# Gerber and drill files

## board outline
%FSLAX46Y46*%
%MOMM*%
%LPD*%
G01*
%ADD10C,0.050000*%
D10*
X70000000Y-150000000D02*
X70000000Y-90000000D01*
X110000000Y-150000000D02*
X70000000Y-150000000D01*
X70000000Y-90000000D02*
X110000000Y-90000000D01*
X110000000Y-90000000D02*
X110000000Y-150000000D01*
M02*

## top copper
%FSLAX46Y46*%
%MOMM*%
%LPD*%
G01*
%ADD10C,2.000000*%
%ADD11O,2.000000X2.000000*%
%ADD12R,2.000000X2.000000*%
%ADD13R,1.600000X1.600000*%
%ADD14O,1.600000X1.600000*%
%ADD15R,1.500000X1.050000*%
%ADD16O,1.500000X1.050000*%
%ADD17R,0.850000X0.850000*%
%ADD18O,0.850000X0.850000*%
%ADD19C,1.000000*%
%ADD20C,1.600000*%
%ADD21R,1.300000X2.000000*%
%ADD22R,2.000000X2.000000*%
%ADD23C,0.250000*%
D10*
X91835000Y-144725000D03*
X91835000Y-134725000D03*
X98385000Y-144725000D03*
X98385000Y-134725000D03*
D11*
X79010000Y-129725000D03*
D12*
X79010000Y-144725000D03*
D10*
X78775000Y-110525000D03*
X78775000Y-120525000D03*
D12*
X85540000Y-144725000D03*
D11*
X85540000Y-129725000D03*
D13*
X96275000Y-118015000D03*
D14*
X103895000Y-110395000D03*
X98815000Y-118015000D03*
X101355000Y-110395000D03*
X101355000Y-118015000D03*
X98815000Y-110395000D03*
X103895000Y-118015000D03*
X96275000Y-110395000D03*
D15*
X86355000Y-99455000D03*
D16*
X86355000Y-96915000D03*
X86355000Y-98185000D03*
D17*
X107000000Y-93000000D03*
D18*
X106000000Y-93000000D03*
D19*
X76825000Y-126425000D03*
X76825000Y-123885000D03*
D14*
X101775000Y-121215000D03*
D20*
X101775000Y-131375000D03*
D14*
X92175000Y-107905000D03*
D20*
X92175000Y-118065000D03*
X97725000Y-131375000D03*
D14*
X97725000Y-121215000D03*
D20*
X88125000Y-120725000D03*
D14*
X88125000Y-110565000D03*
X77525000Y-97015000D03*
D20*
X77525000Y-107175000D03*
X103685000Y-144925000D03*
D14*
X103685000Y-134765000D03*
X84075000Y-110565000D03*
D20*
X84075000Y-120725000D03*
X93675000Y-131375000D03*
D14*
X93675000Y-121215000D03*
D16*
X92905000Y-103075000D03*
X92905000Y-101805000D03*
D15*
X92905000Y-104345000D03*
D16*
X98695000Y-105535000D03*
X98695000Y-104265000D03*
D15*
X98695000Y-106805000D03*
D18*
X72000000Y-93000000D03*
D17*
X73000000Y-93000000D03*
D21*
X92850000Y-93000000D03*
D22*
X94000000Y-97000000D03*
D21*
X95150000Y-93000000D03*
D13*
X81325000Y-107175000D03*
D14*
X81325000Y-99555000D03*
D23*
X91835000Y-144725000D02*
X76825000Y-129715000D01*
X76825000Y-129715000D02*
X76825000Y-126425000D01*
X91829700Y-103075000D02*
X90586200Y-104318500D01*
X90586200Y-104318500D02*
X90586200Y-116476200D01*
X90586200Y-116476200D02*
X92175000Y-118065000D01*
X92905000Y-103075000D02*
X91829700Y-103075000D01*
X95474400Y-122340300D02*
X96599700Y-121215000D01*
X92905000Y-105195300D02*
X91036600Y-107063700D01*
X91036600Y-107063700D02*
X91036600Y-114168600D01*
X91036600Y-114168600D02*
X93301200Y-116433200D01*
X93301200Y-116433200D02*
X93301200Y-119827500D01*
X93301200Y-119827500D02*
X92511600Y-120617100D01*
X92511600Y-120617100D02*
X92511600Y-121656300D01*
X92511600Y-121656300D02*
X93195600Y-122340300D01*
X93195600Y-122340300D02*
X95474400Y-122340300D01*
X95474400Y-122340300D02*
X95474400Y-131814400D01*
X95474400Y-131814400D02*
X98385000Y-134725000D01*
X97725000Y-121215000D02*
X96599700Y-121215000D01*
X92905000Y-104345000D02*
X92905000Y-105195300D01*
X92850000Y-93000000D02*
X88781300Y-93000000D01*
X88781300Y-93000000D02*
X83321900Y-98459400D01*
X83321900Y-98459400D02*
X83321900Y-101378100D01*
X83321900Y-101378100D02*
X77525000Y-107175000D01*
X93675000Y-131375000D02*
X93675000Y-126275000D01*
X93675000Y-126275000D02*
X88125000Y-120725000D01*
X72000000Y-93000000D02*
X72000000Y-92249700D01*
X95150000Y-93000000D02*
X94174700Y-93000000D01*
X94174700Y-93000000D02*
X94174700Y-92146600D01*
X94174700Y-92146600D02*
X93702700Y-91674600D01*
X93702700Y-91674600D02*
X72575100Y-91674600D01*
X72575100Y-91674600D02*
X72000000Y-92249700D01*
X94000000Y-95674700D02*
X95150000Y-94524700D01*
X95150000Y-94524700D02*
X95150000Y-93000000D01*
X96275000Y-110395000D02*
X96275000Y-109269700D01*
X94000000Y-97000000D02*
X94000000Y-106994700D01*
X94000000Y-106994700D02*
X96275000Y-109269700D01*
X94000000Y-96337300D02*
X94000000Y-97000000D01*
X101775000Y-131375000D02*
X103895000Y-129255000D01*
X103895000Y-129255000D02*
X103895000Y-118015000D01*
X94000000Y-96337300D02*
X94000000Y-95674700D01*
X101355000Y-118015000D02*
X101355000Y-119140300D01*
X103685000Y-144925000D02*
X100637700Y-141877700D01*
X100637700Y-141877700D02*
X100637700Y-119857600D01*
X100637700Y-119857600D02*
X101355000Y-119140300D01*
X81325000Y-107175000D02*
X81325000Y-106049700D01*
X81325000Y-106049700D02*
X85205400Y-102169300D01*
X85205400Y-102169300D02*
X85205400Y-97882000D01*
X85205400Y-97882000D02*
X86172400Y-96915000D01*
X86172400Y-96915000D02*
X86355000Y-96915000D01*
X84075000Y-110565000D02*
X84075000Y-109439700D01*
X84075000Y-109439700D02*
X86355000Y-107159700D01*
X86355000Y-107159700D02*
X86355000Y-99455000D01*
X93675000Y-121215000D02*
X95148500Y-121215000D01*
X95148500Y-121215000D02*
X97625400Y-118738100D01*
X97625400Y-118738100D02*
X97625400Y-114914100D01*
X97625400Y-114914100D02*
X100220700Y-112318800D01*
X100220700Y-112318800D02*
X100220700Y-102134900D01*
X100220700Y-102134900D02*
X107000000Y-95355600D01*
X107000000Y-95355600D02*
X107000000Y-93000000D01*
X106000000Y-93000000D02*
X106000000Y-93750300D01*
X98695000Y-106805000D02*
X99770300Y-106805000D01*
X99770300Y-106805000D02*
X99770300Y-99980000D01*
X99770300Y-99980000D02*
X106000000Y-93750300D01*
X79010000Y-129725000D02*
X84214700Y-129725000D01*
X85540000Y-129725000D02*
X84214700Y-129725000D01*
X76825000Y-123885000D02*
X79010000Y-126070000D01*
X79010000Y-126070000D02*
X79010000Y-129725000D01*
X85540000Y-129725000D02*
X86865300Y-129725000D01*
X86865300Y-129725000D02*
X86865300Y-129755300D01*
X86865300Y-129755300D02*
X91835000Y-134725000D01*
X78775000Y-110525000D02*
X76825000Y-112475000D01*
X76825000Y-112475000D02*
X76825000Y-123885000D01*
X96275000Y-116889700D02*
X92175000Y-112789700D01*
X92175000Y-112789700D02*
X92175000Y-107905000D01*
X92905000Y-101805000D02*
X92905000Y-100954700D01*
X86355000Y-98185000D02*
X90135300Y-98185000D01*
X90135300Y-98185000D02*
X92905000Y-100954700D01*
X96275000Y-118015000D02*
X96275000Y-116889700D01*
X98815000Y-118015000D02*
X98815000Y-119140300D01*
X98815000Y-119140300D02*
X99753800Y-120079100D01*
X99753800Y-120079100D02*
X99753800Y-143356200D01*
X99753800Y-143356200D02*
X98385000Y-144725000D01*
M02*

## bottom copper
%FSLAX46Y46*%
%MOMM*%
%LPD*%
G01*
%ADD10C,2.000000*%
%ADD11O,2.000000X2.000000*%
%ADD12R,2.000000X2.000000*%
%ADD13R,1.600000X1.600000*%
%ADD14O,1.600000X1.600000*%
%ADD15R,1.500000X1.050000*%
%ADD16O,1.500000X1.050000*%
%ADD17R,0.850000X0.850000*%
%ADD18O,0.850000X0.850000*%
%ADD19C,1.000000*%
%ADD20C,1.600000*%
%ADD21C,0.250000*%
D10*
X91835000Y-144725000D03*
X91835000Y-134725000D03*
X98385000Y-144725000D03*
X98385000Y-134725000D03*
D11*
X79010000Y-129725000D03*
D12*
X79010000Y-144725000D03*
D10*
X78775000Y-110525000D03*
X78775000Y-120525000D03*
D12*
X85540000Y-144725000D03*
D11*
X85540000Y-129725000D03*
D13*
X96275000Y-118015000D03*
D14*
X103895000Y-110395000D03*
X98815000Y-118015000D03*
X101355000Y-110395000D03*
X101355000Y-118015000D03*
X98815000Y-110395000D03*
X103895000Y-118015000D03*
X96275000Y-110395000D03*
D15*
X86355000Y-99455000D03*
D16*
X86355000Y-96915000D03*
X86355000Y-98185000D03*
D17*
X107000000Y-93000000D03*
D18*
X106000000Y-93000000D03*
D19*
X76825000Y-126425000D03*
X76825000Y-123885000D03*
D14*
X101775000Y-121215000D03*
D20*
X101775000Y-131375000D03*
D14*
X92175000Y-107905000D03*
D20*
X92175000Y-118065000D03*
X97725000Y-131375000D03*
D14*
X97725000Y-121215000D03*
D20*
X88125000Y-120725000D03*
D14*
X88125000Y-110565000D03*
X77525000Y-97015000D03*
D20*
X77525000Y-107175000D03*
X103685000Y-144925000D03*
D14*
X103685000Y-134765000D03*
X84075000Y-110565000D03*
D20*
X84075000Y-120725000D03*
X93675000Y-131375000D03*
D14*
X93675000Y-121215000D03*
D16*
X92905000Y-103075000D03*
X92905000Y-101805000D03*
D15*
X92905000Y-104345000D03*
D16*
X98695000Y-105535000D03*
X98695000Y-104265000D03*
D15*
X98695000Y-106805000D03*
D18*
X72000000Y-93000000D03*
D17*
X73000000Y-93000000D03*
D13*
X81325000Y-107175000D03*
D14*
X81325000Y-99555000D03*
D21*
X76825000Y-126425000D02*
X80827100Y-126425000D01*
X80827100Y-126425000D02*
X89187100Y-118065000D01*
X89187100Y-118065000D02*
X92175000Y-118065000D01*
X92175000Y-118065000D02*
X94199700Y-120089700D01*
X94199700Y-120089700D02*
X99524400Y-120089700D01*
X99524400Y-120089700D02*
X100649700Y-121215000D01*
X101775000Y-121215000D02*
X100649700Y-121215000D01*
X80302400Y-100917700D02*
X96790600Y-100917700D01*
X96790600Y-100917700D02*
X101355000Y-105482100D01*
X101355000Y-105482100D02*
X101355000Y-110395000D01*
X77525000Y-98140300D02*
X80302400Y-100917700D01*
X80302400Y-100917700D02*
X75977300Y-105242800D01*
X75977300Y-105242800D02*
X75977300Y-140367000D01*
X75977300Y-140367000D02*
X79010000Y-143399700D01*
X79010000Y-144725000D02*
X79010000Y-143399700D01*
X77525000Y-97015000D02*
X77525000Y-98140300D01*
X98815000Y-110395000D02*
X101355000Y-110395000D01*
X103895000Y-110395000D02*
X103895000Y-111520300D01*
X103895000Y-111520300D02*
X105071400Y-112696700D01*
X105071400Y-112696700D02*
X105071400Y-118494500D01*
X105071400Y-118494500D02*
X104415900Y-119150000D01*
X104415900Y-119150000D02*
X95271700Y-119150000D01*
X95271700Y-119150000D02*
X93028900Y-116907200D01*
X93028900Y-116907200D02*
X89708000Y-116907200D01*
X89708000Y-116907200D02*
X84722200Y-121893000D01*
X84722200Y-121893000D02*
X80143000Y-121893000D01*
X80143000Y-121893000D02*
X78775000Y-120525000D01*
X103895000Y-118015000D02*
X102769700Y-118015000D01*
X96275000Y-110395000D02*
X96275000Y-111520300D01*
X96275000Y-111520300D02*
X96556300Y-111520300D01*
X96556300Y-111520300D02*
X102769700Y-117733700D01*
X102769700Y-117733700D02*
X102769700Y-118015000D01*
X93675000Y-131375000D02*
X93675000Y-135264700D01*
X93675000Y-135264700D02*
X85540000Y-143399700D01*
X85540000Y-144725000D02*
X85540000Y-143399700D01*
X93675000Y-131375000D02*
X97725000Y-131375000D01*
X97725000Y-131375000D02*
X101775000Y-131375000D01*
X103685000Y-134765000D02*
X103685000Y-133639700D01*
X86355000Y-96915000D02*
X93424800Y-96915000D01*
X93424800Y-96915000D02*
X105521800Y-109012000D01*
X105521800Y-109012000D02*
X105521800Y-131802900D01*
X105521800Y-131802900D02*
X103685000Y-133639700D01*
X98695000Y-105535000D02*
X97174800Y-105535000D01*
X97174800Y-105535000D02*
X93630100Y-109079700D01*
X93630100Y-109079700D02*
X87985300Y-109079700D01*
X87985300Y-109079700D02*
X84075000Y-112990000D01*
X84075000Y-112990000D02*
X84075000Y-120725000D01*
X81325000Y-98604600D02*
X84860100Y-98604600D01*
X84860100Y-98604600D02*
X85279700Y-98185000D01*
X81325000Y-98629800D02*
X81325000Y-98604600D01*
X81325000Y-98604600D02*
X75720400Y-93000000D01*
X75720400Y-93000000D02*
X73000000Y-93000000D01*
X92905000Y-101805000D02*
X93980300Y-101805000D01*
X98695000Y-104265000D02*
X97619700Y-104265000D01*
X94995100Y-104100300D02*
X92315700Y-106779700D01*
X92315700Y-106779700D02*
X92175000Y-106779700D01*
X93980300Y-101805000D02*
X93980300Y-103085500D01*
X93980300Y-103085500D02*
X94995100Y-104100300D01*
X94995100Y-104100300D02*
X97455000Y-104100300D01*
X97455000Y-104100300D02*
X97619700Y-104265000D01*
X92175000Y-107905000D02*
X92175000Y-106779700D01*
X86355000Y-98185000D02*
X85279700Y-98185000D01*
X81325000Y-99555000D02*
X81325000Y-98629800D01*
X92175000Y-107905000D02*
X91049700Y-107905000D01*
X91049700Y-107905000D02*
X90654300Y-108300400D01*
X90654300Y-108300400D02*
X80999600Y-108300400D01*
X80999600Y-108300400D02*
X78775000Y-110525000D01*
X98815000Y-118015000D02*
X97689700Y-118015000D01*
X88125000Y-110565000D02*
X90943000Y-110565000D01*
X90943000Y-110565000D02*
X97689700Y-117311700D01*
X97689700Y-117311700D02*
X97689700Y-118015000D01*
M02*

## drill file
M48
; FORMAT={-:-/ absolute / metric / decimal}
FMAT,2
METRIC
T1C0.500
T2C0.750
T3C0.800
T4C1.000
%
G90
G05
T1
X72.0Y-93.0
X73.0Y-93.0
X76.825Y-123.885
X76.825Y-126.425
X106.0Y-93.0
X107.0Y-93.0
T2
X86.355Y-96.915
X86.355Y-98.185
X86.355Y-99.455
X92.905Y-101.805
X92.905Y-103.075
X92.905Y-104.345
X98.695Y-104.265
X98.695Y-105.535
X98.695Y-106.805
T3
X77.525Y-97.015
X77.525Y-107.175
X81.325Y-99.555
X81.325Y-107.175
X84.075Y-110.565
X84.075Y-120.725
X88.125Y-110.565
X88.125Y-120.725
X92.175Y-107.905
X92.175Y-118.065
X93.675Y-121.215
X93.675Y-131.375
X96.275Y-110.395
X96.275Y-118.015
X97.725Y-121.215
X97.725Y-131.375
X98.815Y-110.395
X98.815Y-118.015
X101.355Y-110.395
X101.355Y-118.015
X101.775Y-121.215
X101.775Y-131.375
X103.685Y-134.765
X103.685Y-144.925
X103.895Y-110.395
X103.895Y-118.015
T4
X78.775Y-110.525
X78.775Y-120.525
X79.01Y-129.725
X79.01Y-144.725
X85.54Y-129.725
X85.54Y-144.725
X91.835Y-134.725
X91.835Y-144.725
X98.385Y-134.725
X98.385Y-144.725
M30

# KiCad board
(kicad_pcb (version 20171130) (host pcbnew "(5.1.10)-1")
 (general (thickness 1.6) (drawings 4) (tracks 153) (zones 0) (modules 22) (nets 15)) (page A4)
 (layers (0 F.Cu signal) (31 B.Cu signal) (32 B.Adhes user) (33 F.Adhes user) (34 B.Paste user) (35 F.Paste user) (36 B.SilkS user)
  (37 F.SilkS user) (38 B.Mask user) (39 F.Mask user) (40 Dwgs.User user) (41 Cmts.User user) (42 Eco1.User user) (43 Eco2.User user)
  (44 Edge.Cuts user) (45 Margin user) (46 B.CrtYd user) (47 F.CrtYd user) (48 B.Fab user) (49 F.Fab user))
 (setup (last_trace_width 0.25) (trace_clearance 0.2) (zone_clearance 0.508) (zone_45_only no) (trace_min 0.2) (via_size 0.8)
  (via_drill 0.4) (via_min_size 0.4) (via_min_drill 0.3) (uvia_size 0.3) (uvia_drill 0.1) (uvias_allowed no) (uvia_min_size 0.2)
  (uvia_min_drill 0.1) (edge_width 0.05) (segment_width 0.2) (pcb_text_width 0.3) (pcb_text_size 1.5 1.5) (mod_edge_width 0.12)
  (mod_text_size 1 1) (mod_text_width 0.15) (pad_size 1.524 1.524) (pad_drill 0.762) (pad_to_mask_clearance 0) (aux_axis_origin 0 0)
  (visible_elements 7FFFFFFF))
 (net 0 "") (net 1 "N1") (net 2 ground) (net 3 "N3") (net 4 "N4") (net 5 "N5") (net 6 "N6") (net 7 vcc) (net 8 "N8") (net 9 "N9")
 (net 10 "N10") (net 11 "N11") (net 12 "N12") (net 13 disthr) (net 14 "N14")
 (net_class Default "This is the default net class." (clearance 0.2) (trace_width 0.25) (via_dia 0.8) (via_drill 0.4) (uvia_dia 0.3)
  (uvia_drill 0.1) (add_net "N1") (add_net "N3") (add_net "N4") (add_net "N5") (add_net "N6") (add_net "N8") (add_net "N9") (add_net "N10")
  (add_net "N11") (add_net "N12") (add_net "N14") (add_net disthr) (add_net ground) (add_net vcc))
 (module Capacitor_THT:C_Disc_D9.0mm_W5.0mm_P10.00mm (layer F.Cu) (at 91.835 144.725 90)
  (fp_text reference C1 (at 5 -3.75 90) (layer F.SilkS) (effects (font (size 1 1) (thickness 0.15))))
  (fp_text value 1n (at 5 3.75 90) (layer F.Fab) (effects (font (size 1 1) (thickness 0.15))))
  (pad 1 thru_hole circle (at 0 0 90) (size 2 2) (drill 1) (layers *.Cu *.Mask) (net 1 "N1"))
  (pad 2 thru_hole circle (at 10 0 90) (size 2 2) (drill 1) (layers *.Cu *.Mask) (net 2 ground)))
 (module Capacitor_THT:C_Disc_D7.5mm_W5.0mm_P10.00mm (layer F.Cu) (at 98.385 144.725 90)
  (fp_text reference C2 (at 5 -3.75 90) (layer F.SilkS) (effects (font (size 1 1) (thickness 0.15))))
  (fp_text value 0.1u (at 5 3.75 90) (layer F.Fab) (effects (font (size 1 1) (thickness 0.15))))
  (pad 1 thru_hole circle (at 0 0 90) (size 2 2) (drill 1) (layers *.Cu *.Mask) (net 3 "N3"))
  (pad 2 thru_hole circle (at 10 0 90) (size 2 2) (drill 1) (layers *.Cu *.Mask) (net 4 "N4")))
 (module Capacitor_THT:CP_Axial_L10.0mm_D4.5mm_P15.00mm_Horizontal (layer F.Cu) (at 79.01 144.725 90)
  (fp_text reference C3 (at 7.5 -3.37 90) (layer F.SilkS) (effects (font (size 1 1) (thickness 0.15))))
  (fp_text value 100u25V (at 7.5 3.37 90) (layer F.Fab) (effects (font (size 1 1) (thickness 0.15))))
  (pad 2 thru_hole oval (at 15 0 90) (size 2 2) (drill 1) (layers *.Cu *.Mask) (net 2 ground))
  (pad 1 thru_hole rect (at 0 0 90) (size 2 2) (drill 1) (layers *.Cu *.Mask) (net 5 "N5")))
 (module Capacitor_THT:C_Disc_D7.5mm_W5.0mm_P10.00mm (layer F.Cu) (at 78.775 120.525 90)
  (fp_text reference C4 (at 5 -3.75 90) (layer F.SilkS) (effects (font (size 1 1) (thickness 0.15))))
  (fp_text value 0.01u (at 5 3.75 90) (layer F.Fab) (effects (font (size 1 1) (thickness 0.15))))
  (pad 2 thru_hole circle (at 10 0 90) (size 2 2) (drill 1) (layers *.Cu *.Mask) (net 2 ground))
  (pad 1 thru_hole circle (at 0 0 90) (size 2 2) (drill 1) (layers *.Cu *.Mask) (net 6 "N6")))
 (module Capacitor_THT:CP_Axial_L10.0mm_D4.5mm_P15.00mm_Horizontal (layer F.Cu) (at 85.54 144.725 90)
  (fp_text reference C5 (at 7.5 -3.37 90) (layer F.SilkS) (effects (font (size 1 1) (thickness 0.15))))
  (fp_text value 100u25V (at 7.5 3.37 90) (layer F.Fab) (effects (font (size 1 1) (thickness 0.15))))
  (pad 1 thru_hole rect (at 0 0 90) (size 2 2) (drill 1) (layers *.Cu *.Mask) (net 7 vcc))
  (pad 2 thru_hole oval (at 15 0 90) (size 2 2) (drill 1) (layers *.Cu *.Mask) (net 2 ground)))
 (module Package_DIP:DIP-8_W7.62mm (layer F.Cu) (at 96.275 118.015 90)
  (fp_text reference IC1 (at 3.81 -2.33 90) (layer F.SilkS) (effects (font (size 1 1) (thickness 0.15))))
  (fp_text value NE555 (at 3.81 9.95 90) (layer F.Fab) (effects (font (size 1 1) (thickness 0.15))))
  (pad 1 thru_hole rect (at 0 0 90) (size 1.6 1.6) (drill 0.8) (layers *.Cu *.Mask) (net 2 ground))
  (pad 5 thru_hole oval (at 7.62 7.62 90) (size 1.6 1.6) (drill 0.8) (layers *.Cu *.Mask) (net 6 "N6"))
  (pad 2 thru_hole oval (at 0 2.54 90) (size 1.6 1.6) (drill 0.8) (layers *.Cu *.Mask) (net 3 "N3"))
  (pad 6 thru_hole oval (at 7.62 5.08 90) (size 1.6 1.6) (drill 0.8) (layers *.Cu *.Mask) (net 5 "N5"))
  (pad 3 thru_hole oval (at 0 5.08 90) (size 1.6 1.6) (drill 0.8) (layers *.Cu *.Mask) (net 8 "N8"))
  (pad 7 thru_hole oval (at 7.62 2.54 90) (size 1.6 1.6) (drill 0.8) (layers *.Cu *.Mask) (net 5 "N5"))
  (pad 4 thru_hole oval (at 0 7.62 90) (size 1.6 1.6) (drill 0.8) (layers *.Cu *.Mask) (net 7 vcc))
  (pad 8 thru_hole oval (at 7.62 0 90) (size 1.6 1.6) (drill 0.8) (layers *.Cu *.Mask) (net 7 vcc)))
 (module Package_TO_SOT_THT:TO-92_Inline (layer F.Cu) (at 86.355 99.455 90)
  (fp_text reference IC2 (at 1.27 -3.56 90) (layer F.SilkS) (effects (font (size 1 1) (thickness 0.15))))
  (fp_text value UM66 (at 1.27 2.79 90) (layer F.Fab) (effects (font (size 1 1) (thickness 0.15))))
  (pad 1 thru_hole rect (at 0 0 90) (size 1.05 1.5) (drill 0.75) (layers *.Cu *.Mask) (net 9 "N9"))
  (pad 3 thru_hole oval (at 2.54 0 90) (size 1.05 1.5) (drill 0.75) (layers *.Cu *.Mask) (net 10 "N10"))
  (pad 2 thru_hole oval (at 1.27 0 90) (size 1.05 1.5) (drill 0.75) (layers *.Cu *.Mask) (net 2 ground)))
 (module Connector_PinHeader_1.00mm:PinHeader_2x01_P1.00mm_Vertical (layer F.Cu) (at 107 93 180)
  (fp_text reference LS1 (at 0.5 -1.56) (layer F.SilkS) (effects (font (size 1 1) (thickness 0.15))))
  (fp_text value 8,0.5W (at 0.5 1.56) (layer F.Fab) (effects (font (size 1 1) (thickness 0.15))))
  (pad 1 thru_hole rect (at 0 0 180) (size 0.85 0.85) (drill 0.5) (layers *.Cu *.Mask) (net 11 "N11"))
  (pad 2 thru_hole oval (at 1 0 180) (size 0.85 0.85) (drill 0.5) (layers *.Cu *.Mask) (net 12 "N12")))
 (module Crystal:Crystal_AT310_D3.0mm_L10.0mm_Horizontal (layer F.Cu) (at 76.825 126.425 90)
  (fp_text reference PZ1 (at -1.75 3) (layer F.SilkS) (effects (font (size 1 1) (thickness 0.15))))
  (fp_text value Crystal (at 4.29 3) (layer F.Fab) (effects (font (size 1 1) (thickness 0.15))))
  (pad 1 thru_hole circle (at 0 0 90) (size 1 1) (drill 0.5) (layers *.Cu *.Mask) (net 1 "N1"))
  (pad 2 thru_hole circle (at 2.54 0 90) (size 1 1) (drill 0.5) (layers *.Cu *.Mask) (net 2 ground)))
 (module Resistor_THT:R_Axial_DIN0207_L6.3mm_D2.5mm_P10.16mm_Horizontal (layer F.Cu) (at 101.775 131.375 90)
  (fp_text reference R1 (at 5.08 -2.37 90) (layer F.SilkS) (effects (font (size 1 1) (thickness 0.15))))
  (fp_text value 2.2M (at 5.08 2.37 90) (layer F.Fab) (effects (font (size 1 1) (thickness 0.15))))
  (pad 2 thru_hole oval (at 10.16 0 90) (size 1.6 1.6) (drill 0.8) (layers *.Cu *.Mask) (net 1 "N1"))
  (pad 1 thru_hole circle (at 0 0 90) (size 1.6 1.6) (drill 0.8) (layers *.Cu *.Mask) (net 7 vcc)))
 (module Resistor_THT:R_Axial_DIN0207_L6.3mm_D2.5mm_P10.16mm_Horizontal (layer F.Cu) (at 92.175 118.065 90)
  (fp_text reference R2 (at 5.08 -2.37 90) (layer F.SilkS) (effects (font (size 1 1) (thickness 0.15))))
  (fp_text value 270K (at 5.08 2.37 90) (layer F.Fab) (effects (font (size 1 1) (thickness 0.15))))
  (pad 2 thru_hole oval (at 10.16 0 90) (size 1.6 1.6) (drill 0.8) (layers *.Cu *.Mask) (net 2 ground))
  (pad 1 thru_hole circle (at 0 0 90) (size 1.6 1.6) (drill 0.8) (layers *.Cu *.Mask) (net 1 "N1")))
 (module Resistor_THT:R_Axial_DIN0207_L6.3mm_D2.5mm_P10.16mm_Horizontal (layer F.Cu) (at 97.725 131.375 90)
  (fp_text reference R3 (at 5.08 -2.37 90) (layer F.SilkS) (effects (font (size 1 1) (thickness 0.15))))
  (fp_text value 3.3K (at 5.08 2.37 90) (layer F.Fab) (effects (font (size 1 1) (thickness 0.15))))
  (pad 1 thru_hole circle (at 0 0 90) (size 1.6 1.6) (drill 0.8) (layers *.Cu *.Mask) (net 7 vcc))
  (pad 2 thru_hole oval (at 10.16 0 90) (size 1.6 1.6) (drill 0.8) (layers *.Cu *.Mask) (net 4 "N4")))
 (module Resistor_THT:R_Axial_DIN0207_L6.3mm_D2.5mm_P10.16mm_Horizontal (layer F.Cu) (at 88.125 120.725 90)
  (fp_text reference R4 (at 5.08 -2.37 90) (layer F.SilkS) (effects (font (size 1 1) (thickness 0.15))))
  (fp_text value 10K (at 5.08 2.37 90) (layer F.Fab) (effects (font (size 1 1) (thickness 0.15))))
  (pad 1 thru_hole circle (at 0 0 90) (size 1.6 1.6) (drill 0.8) (layers *.Cu *.Mask) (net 7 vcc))
  (pad 2 thru_hole oval (at 10.16 0 90) (size 1.6 1.6) (drill 0.8) (layers *.Cu *.Mask) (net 3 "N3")))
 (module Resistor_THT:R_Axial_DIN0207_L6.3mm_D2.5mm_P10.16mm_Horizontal (layer F.Cu) (at 77.525 107.175 90)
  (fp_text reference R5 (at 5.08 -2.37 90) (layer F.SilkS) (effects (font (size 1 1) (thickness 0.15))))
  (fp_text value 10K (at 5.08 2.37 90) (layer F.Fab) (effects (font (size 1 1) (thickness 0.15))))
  (pad 2 thru_hole oval (at 10.16 0 90) (size 1.6 1.6) (drill 0.8) (layers *.Cu *.Mask) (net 5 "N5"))
  (pad 1 thru_hole circle (at 0 0 90) (size 1.6 1.6) (drill 0.8) (layers *.Cu *.Mask) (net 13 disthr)))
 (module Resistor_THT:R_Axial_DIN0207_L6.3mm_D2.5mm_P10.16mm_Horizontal (layer F.Cu) (at 103.685 144.925 90)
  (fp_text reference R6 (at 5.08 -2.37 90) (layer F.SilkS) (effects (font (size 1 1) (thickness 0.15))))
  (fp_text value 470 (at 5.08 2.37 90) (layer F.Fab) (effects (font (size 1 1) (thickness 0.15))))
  (pad 1 thru_hole circle (at 0 0 90) (size 1.6 1.6) (drill 0.8) (layers *.Cu *.Mask) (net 8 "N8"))
  (pad 2 thru_hole oval (at 10.16 0 90) (size 1.6 1.6) (drill 0.8) (layers *.Cu *.Mask) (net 10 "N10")))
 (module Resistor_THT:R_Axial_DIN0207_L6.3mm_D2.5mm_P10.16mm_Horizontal (layer F.Cu) (at 84.075 120.725 90)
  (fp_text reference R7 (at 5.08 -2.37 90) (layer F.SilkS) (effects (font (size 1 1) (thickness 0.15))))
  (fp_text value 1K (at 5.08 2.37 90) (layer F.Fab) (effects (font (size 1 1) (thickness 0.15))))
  (pad 2 thru_hole oval (at 10.16 0 90) (size 1.6 1.6) (drill 0.8) (layers *.Cu *.Mask) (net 9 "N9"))
  (pad 1 thru_hole circle (at 0 0 90) (size 1.6 1.6) (drill 0.8) (layers *.Cu *.Mask) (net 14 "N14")))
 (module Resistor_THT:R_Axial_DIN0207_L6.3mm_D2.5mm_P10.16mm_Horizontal (layer F.Cu) (at 93.675 131.375 90)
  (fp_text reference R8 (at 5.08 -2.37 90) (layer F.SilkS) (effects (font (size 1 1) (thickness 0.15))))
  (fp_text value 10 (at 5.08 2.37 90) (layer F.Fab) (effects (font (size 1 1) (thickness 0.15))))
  (pad 1 thru_hole circle (at 0 0 90) (size 1.6 1.6) (drill 0.8) (layers *.Cu *.Mask) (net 7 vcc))
  (pad 2 thru_hole oval (at 10.16 0 90) (size 1.6 1.6) (drill 0.8) (layers *.Cu *.Mask) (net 11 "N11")))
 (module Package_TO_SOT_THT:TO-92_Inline (layer F.Cu) (at 92.905 104.345 90)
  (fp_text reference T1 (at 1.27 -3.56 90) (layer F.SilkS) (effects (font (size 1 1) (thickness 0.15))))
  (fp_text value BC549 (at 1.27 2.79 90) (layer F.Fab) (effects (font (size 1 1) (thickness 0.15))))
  (pad 2 thru_hole oval (at 1.27 0 90) (size 1.05 1.5) (drill 0.75) (layers *.Cu *.Mask) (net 1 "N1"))
  (pad 3 thru_hole oval (at 2.54 0 90) (size 1.05 1.5) (drill 0.75) (layers *.Cu *.Mask) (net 2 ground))
  (pad 1 thru_hole rect (at 0 0 90) (size 1.05 1.5) (drill 0.75) (layers *.Cu *.Mask) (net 4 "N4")))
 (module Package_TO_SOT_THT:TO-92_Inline (layer F.Cu) (at 98.695 106.805 90)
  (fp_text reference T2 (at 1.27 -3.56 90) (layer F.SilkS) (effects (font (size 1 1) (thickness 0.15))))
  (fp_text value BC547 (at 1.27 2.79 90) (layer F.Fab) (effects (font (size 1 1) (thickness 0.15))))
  (pad 2 thru_hole oval (at 1.27 0 90) (size 1.05 1.5) (drill 0.75) (layers *.Cu *.Mask) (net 14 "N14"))
  (pad 3 thru_hole oval (at 2.54 0 90) (size 1.05 1.5) (drill 0.75) (layers *.Cu *.Mask) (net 2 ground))
  (pad 1 thru_hole rect (at 0 0 90) (size 1.05 1.5) (drill 0.75) (layers *.Cu *.Mask) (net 12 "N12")))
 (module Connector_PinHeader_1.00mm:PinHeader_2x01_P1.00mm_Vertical (layer F.Cu) (at 73 93 180)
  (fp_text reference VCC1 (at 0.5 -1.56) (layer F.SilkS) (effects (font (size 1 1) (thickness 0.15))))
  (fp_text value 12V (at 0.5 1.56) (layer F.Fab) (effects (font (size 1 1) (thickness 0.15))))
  (pad 2 thru_hole oval (at 1 0 180) (size 0.85 0.85) (drill 0.5) (layers *.Cu *.Mask) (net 7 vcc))
  (pad 1 thru_hole rect (at 0 0 180) (size 0.85 0.85) (drill 0.5) (layers *.Cu *.Mask) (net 2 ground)))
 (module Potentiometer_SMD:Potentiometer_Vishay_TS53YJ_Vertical (layer F.Cu) (at 94 95 90)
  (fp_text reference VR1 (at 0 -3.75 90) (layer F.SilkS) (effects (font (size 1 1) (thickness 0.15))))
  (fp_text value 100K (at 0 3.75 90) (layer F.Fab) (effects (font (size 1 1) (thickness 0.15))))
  (pad 1 smd rect (at 2 -1.15 90) (size 2 1.3) (layers F.Cu F.Paste F.Mask) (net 13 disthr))
  (pad 2 smd rect (at -2 0 90) (size 2 2) (layers F.Cu F.Paste F.Mask) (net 7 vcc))
  (pad 3 smd rect (at 2 1.15 90) (size 2 1.3) (layers F.Cu F.Paste F.Mask) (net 7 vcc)))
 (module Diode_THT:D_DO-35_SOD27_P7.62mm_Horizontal (layer F.Cu) (at 81.325 107.175 90)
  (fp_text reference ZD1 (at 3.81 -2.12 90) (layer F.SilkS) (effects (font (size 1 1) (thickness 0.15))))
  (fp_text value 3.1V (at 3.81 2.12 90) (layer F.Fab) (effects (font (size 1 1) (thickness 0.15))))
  (pad 1 thru_hole rect (at 0 0 90) (size 1.6 1.6) (drill 0.8) (layers *.Cu *.Mask) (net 10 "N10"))
  (pad 2 thru_hole oval (at 7.62 0 90) (size 1.6 1.6) (drill 0.8) (layers *.Cu *.Mask) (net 2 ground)))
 (gr_line (start 70 150) (end 70 90) (layer Edge.Cuts) (width 0.05))
 (gr_line (start 110 150) (end 70 150) (layer Edge.Cuts) (width 0.05))
 (gr_line (start 70 90) (end 110 90) (layer Edge.Cuts) (width 0.05))
 (gr_line (start 110 90) (end 110 150) (layer Edge.Cuts) (width 0.05))
 (segment (start 76.825 126.425) (end 80.8271 126.425) (width 0.25) (layer B.Cu) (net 1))
 (segment (start 80.8271 126.425) (end 89.1871 118.065) (width 0.25) (layer B.Cu) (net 1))
 (segment (start 89.1871 118.065) (end 92.175 118.065) (width 0.25) (layer B.Cu) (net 1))
 (segment (start 92.175 118.065) (end 94.1997 120.0897) (width 0.25) (layer B.Cu) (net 1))
 (segment (start 94.1997 120.0897) (end 99.5244 120.0897) (width 0.25) (layer B.Cu) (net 1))
 (segment (start 99.5244 120.0897) (end 100.6497 121.215) (width 0.25) (layer B.Cu) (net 1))
 (segment (start 101.775 121.215) (end 100.6497 121.215) (width 0.25) (layer B.Cu) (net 1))
 (segment (start 91.835 144.725) (end 76.825 129.715) (width 0.25) (layer F.Cu) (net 1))
 (segment (start 76.825 129.715) (end 76.825 126.425) (width 0.25) (layer F.Cu) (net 1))
 (segment (start 91.8297 103.075) (end 90.5862 104.3185) (width 0.25) (layer F.Cu) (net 1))
 (segment (start 90.5862 104.3185) (end 90.5862 116.4762) (width 0.25) (layer F.Cu) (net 1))
 (segment (start 90.5862 116.4762) (end 92.175 118.065) (width 0.25) (layer F.Cu) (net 1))
 (segment (start 92.905 103.075) (end 91.8297 103.075) (width 0.25) (layer F.Cu) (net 1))
 (segment (start 95.4744 122.3403) (end 96.5997 121.215) (width 0.25) (layer F.Cu) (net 4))
 (segment (start 92.905 105.1953) (end 91.0366 107.0637) (width 0.25) (layer F.Cu) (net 4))
 (segment (start 91.0366 107.0637) (end 91.0366 114.1686) (width 0.25) (layer F.Cu) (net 4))
 (segment (start 91.0366 114.1686) (end 93.3012 116.4332) (width 0.25) (layer F.Cu) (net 4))
 (segment (start 93.3012 116.4332) (end 93.3012 119.8275) (width 0.25) (layer F.Cu) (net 4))
 (segment (start 93.3012 119.8275) (end 92.5116 120.6171) (width 0.25) (layer F.Cu) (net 4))
 (segment (start 92.5116 120.6171) (end 92.5116 121.6563) (width 0.25) (layer F.Cu) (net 4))
 (segment (start 92.5116 121.6563) (end 93.1956 122.3403) (width 0.25) (layer F.Cu) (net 4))
 (segment (start 93.1956 122.3403) (end 95.4744 122.3403) (width 0.25) (layer F.Cu) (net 4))
 (segment (start 95.4744 122.3403) (end 95.4744 131.8144) (width 0.25) (layer F.Cu) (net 4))
 (segment (start 95.4744 131.8144) (end 98.385 134.725) (width 0.25) (layer F.Cu) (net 4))
 (segment (start 97.725 121.215) (end 96.5997 121.215) (width 0.25) (layer F.Cu) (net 4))
 (segment (start 92.905 104.345) (end 92.905 105.1953) (width 0.25) (layer F.Cu) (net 4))
 (segment (start 92.85 93) (end 88.7813 93) (width 0.25) (layer F.Cu) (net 13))
 (segment (start 88.7813 93) (end 83.3219 98.4594) (width 0.25) (layer F.Cu) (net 13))
 (segment (start 83.3219 98.4594) (end 83.3219 101.3781) (width 0.25) (layer F.Cu) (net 13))
 (segment (start 83.3219 101.3781) (end 77.525 107.175) (width 0.25) (layer F.Cu) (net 13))
 (segment (start 80.3024 100.9177) (end 96.7906 100.9177) (width 0.25) (layer B.Cu) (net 5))
 (segment (start 96.7906 100.9177) (end 101.355 105.4821) (width 0.25) (layer B.Cu) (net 5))
 (segment (start 101.355 105.4821) (end 101.355 110.395) (width 0.25) (layer B.Cu) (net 5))
 (segment (start 77.525 98.1403) (end 80.3024 100.9177) (width 0.25) (layer B.Cu) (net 5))
 (segment (start 80.3024 100.9177) (end 75.9773 105.2428) (width 0.25) (layer B.Cu) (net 5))
 (segment (start 75.9773 105.2428) (end 75.9773 140.367) (width 0.25) (layer B.Cu) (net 5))
 (segment (start 75.9773 140.367) (end 79.01 143.3997) (width 0.25) (layer B.Cu) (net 5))
 (segment (start 79.01 144.725) (end 79.01 143.3997) (width 0.25) (layer B.Cu) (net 5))
 (segment (start 77.525 97.015) (end 77.525 98.1403) (width 0.25) (layer B.Cu) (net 5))
 (segment (start 98.815 110.395) (end 101.355 110.395) (width 0.25) (layer B.Cu) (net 5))
 (segment (start 103.895 110.395) (end 103.895 111.5203) (width 0.25) (layer B.Cu) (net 6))
 (segment (start 103.895 111.5203) (end 105.0714 112.6967) (width 0.25) (layer B.Cu) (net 6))
 (segment (start 105.0714 112.6967) (end 105.0714 118.4945) (width 0.25) (layer B.Cu) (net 6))
 (segment (start 105.0714 118.4945) (end 104.4159 119.15) (width 0.25) (layer B.Cu) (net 6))
 (segment (start 104.4159 119.15) (end 95.2717 119.15) (width 0.25) (layer B.Cu) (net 6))
 (segment (start 95.2717 119.15) (end 93.0289 116.9072) (width 0.25) (layer B.Cu) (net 6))
 (segment (start 93.0289 116.9072) (end 89.708 116.9072) (width 0.25) (layer B.Cu) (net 6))
 (segment (start 89.708 116.9072) (end 84.7222 121.893) (width 0.25) (layer B.Cu) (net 6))
 (segment (start 84.7222 121.893) (end 80.143 121.893) (width 0.25) (layer B.Cu) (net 6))
 (segment (start 80.143 121.893) (end 78.775 120.525) (width 0.25) (layer B.Cu) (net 6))
 (segment (start 93.675 131.375) (end 93.675 126.275) (width 0.25) (layer F.Cu) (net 7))
 (segment (start 93.675 126.275) (end 88.125 120.725) (width 0.25) (layer F.Cu) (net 7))
 (segment (start 103.895 118.015) (end 102.7697 118.015) (width 0.25) (layer B.Cu) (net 7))
 (segment (start 96.275 110.395) (end 96.275 111.5203) (width 0.25) (layer B.Cu) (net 7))
 (segment (start 96.275 111.5203) (end 96.5563 111.5203) (width 0.25) (layer B.Cu) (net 7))
 (segment (start 96.5563 111.5203) (end 102.7697 117.7337) (width 0.25) (layer B.Cu) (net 7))
 (segment (start 102.7697 117.7337) (end 102.7697 118.015) (width 0.25) (layer B.Cu) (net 7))
 (segment (start 93.675 131.375) (end 93.675 135.2647) (width 0.25) (layer B.Cu) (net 7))
 (segment (start 93.675 135.2647) (end 85.54 143.3997) (width 0.25) (layer B.Cu) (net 7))
 (segment (start 85.54 144.725) (end 85.54 143.3997) (width 0.25) (layer B.Cu) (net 7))
 (segment (start 93.675 131.375) (end 97.725 131.375) (width 0.25) (layer B.Cu) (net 7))
 (segment (start 72 93) (end 72 92.2497) (width 0.25) (layer F.Cu) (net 7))
 (segment (start 95.15 93) (end 94.1747 93) (width 0.25) (layer F.Cu) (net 7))
 (segment (start 94.1747 93) (end 94.1747 92.1466) (width 0.25) (layer F.Cu) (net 7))
 (segment (start 94.1747 92.1466) (end 93.7027 91.6746) (width 0.25) (layer F.Cu) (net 7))
 (segment (start 93.7027 91.6746) (end 72.5751 91.6746) (width 0.25) (layer F.Cu) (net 7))
 (segment (start 72.5751 91.6746) (end 72 92.2497) (width 0.25) (layer F.Cu) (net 7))
 (segment (start 94 95.6747) (end 95.15 94.5247) (width 0.25) (layer F.Cu) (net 7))
 (segment (start 95.15 94.5247) (end 95.15 93) (width 0.25) (layer F.Cu) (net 7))
 (segment (start 96.275 110.395) (end 96.275 109.2697) (width 0.25) (layer F.Cu) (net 7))
 (segment (start 94 97) (end 94 106.9947) (width 0.25) (layer F.Cu) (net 7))
 (segment (start 94 106.9947) (end 96.275 109.2697) (width 0.25) (layer F.Cu) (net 7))
 (segment (start 94 96.3373) (end 94 97) (width 0.25) (layer F.Cu) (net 7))
 (segment (start 101.775 131.375) (end 103.895 129.255) (width 0.25) (layer F.Cu) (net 7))
 (segment (start 103.895 129.255) (end 103.895 118.015) (width 0.25) (layer F.Cu) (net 7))
 (segment (start 97.725 131.375) (end 101.775 131.375) (width 0.25) (layer B.Cu) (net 7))
 (segment (start 94 96.3373) (end 94 95.6747) (width 0.25) (layer F.Cu) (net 7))
 (segment (start 101.355 118.015) (end 101.355 119.1403) (width 0.25) (layer F.Cu) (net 8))
 (segment (start 103.685 144.925) (end 100.6377 141.8777) (width 0.25) (layer F.Cu) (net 8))
 (segment (start 100.6377 141.8777) (end 100.6377 119.8576) (width 0.25) (layer F.Cu) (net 8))
 (segment (start 100.6377 119.8576) (end 101.355 119.1403) (width 0.25) (layer F.Cu) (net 8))
 (segment (start 103.685 134.765) (end 103.685 133.6397) (width 0.25) (layer B.Cu) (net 10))
 (segment (start 86.355 96.915) (end 93.4248 96.915) (width 0.25) (layer B.Cu) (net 10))
 (segment (start 93.4248 96.915) (end 105.5218 109.012) (width 0.25) (layer B.Cu) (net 10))
 (segment (start 105.5218 109.012) (end 105.5218 131.8029) (width 0.25) (layer B.Cu) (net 10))
 (segment (start 105.5218 131.8029) (end 103.685 133.6397) (width 0.25) (layer B.Cu) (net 10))
 (segment (start 81.325 107.175) (end 81.325 106.0497) (width 0.25) (layer F.Cu) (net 10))
 (segment (start 81.325 106.0497) (end 85.2054 102.1693) (width 0.25) (layer F.Cu) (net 10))
 (segment (start 85.2054 102.1693) (end 85.2054 97.882) (width 0.25) (layer F.Cu) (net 10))
 (segment (start 85.2054 97.882) (end 86.1724 96.915) (width 0.25) (layer F.Cu) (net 10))
 (segment (start 86.1724 96.915) (end 86.355 96.915) (width 0.25) (layer F.Cu) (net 10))
 (segment (start 84.075 110.565) (end 84.075 109.4397) (width 0.25) (layer F.Cu) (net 9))
 (segment (start 84.075 109.4397) (end 86.355 107.1597) (width 0.25) (layer F.Cu) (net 9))
 (segment (start 86.355 107.1597) (end 86.355 99.455) (width 0.25) (layer F.Cu) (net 9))
 (segment (start 93.675 121.215) (end 95.1485 121.215) (width 0.25) (layer F.Cu) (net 11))
 (segment (start 95.1485 121.215) (end 97.6254 118.7381) (width 0.25) (layer F.Cu) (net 11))
 (segment (start 97.6254 118.7381) (end 97.6254 114.9141) (width 0.25) (layer F.Cu) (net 11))
 (segment (start 97.6254 114.9141) (end 100.2207 112.3188) (width 0.25) (layer F.Cu) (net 11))
 (segment (start 100.2207 112.3188) (end 100.2207 102.1349) (width 0.25) (layer F.Cu) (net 11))
 (segment (start 100.2207 102.1349) (end 107 95.3556) (width 0.25) (layer F.Cu) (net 11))
 (segment (start 107 95.3556) (end 107 93) (width 0.25) (layer F.Cu) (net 11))
 (segment (start 106 93) (end 106 93.7503) (width 0.25) (layer F.Cu) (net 12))
 (segment (start 98.695 106.805) (end 99.7703 106.805) (width 0.25) (layer F.Cu) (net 12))
 (segment (start 99.7703 106.805) (end 99.7703 99.98) (width 0.25) (layer F.Cu) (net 12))
 (segment (start 99.7703 99.98) (end 106 93.7503) (width 0.25) (layer F.Cu) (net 12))
 (segment (start 98.695 105.535) (end 97.1748 105.535) (width 0.25) (layer B.Cu) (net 14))
 (segment (start 97.1748 105.535) (end 93.6301 109.0797) (width 0.25) (layer B.Cu) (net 14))
 (segment (start 93.6301 109.0797) (end 87.9853 109.0797) (width 0.25) (layer B.Cu) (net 14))
 (segment (start 87.9853 109.0797) (end 84.075 112.99) (width 0.25) (layer B.Cu) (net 14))
 (segment (start 84.075 112.99) (end 84.075 120.725) (width 0.25) (layer B.Cu) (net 14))
 (segment (start 79.01 129.725) (end 84.2147 129.725) (width 0.25) (layer F.Cu) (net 2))
 (segment (start 85.54 129.725) (end 84.2147 129.725) (width 0.25) (layer F.Cu) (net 2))
 (segment (start 76.825 123.885) (end 79.01 126.07) (width 0.25) (layer F.Cu) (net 2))
 (segment (start 79.01 126.07) (end 79.01 129.725) (width 0.25) (layer F.Cu) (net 2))
 (segment (start 85.54 129.725) (end 86.8653 129.725) (width 0.25) (layer F.Cu) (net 2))
 (segment (start 86.8653 129.725) (end 86.8653 129.7553) (width 0.25) (layer F.Cu) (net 2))
 (segment (start 86.8653 129.7553) (end 91.835 134.725) (width 0.25) (layer F.Cu) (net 2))
 (segment (start 81.325 98.6046) (end 84.8601 98.6046) (width 0.25) (layer B.Cu) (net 2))
 (segment (start 84.8601 98.6046) (end 85.2797 98.185) (width 0.25) (layer B.Cu) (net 2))
 (segment (start 81.325 98.6298) (end 81.325 98.6046) (width 0.25) (layer B.Cu) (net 2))
 (segment (start 81.325 98.6046) (end 75.7204 93) (width 0.25) (layer B.Cu) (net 2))
 (segment (start 75.7204 93) (end 73 93) (width 0.25) (layer B.Cu) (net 2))
 (segment (start 78.775 110.525) (end 76.825 112.475) (width 0.25) (layer F.Cu) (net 2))
 (segment (start 76.825 112.475) (end 76.825 123.885) (width 0.25) (layer F.Cu) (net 2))
 (segment (start 96.275 116.8897) (end 92.175 112.7897) (width 0.25) (layer F.Cu) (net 2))
 (segment (start 92.175 112.7897) (end 92.175 107.905) (width 0.25) (layer F.Cu) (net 2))
 (segment (start 92.905 101.805) (end 93.9803 101.805) (width 0.25) (layer B.Cu) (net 2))
 (segment (start 98.695 104.265) (end 97.6197 104.265) (width 0.25) (layer B.Cu) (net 2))
 (segment (start 94.9951 104.1003) (end 92.3157 106.7797) (width 0.25) (layer B.Cu) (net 2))
 (segment (start 92.3157 106.7797) (end 92.175 106.7797) (width 0.25) (layer B.Cu) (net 2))
 (segment (start 93.9803 101.805) (end 93.9803 103.0855) (width 0.25) (layer B.Cu) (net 2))
 (segment (start 93.9803 103.0855) (end 94.9951 104.1003) (width 0.25) (layer B.Cu) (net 2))
 (segment (start 94.9951 104.1003) (end 97.455 104.1003) (width 0.25) (layer B.Cu) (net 2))
 (segment (start 97.455 104.1003) (end 97.6197 104.265) (width 0.25) (layer B.Cu) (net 2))
 (segment (start 92.175 107.905) (end 92.175 106.7797) (width 0.25) (layer B.Cu) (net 2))
 (segment (start 86.355 98.185) (end 85.2797 98.185) (width 0.25) (layer B.Cu) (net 2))
 (segment (start 81.325 99.555) (end 81.325 98.6298) (width 0.25) (layer B.Cu) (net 2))
 (segment (start 92.175 107.905) (end 91.0497 107.905) (width 0.25) (layer B.Cu) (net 2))
 (segment (start 91.0497 107.905) (end 90.6543 108.3004) (width 0.25) (layer B.Cu) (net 2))
 (segment (start 90.6543 108.3004) (end 80.9996 108.3004) (width 0.25) (layer B.Cu) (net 2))
 (segment (start 80.9996 108.3004) (end 78.775 110.525) (width 0.25) (layer B.Cu) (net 2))
 (segment (start 92.905 101.805) (end 92.905 100.9547) (width 0.25) (layer F.Cu) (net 2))
 (segment (start 86.355 98.185) (end 90.1353 98.185) (width 0.25) (layer F.Cu) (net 2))
 (segment (start 90.1353 98.185) (end 92.905 100.9547) (width 0.25) (layer F.Cu) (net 2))
 (segment (start 96.275 118.015) (end 96.275 116.8897) (width 0.25) (layer F.Cu) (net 2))
 (segment (start 98.815 118.015) (end 97.6897 118.015) (width 0.25) (layer B.Cu) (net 3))
 (segment (start 88.125 110.565) (end 90.943 110.565) (width 0.25) (layer B.Cu) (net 3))
 (segment (start 90.943 110.565) (end 97.6897 117.3117) (width 0.25) (layer B.Cu) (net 3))
 (segment (start 97.6897 117.3117) (end 97.6897 118.015) (width 0.25) (layer B.Cu) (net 3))
 (segment (start 98.815 118.015) (end 98.815 119.1403) (width 0.25) (layer F.Cu) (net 3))
 (segment (start 98.815 119.1403) (end 99.7538 120.0791) (width 0.25) (layer F.Cu) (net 3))
 (segment (start 99.7538 120.0791) (end 99.7538 143.3562) (width 0.25) (layer F.Cu) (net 3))
 (segment (start 99.7538 143.3562) (end 98.385 144.725) (width 0.25) (layer F.Cu) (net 3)))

